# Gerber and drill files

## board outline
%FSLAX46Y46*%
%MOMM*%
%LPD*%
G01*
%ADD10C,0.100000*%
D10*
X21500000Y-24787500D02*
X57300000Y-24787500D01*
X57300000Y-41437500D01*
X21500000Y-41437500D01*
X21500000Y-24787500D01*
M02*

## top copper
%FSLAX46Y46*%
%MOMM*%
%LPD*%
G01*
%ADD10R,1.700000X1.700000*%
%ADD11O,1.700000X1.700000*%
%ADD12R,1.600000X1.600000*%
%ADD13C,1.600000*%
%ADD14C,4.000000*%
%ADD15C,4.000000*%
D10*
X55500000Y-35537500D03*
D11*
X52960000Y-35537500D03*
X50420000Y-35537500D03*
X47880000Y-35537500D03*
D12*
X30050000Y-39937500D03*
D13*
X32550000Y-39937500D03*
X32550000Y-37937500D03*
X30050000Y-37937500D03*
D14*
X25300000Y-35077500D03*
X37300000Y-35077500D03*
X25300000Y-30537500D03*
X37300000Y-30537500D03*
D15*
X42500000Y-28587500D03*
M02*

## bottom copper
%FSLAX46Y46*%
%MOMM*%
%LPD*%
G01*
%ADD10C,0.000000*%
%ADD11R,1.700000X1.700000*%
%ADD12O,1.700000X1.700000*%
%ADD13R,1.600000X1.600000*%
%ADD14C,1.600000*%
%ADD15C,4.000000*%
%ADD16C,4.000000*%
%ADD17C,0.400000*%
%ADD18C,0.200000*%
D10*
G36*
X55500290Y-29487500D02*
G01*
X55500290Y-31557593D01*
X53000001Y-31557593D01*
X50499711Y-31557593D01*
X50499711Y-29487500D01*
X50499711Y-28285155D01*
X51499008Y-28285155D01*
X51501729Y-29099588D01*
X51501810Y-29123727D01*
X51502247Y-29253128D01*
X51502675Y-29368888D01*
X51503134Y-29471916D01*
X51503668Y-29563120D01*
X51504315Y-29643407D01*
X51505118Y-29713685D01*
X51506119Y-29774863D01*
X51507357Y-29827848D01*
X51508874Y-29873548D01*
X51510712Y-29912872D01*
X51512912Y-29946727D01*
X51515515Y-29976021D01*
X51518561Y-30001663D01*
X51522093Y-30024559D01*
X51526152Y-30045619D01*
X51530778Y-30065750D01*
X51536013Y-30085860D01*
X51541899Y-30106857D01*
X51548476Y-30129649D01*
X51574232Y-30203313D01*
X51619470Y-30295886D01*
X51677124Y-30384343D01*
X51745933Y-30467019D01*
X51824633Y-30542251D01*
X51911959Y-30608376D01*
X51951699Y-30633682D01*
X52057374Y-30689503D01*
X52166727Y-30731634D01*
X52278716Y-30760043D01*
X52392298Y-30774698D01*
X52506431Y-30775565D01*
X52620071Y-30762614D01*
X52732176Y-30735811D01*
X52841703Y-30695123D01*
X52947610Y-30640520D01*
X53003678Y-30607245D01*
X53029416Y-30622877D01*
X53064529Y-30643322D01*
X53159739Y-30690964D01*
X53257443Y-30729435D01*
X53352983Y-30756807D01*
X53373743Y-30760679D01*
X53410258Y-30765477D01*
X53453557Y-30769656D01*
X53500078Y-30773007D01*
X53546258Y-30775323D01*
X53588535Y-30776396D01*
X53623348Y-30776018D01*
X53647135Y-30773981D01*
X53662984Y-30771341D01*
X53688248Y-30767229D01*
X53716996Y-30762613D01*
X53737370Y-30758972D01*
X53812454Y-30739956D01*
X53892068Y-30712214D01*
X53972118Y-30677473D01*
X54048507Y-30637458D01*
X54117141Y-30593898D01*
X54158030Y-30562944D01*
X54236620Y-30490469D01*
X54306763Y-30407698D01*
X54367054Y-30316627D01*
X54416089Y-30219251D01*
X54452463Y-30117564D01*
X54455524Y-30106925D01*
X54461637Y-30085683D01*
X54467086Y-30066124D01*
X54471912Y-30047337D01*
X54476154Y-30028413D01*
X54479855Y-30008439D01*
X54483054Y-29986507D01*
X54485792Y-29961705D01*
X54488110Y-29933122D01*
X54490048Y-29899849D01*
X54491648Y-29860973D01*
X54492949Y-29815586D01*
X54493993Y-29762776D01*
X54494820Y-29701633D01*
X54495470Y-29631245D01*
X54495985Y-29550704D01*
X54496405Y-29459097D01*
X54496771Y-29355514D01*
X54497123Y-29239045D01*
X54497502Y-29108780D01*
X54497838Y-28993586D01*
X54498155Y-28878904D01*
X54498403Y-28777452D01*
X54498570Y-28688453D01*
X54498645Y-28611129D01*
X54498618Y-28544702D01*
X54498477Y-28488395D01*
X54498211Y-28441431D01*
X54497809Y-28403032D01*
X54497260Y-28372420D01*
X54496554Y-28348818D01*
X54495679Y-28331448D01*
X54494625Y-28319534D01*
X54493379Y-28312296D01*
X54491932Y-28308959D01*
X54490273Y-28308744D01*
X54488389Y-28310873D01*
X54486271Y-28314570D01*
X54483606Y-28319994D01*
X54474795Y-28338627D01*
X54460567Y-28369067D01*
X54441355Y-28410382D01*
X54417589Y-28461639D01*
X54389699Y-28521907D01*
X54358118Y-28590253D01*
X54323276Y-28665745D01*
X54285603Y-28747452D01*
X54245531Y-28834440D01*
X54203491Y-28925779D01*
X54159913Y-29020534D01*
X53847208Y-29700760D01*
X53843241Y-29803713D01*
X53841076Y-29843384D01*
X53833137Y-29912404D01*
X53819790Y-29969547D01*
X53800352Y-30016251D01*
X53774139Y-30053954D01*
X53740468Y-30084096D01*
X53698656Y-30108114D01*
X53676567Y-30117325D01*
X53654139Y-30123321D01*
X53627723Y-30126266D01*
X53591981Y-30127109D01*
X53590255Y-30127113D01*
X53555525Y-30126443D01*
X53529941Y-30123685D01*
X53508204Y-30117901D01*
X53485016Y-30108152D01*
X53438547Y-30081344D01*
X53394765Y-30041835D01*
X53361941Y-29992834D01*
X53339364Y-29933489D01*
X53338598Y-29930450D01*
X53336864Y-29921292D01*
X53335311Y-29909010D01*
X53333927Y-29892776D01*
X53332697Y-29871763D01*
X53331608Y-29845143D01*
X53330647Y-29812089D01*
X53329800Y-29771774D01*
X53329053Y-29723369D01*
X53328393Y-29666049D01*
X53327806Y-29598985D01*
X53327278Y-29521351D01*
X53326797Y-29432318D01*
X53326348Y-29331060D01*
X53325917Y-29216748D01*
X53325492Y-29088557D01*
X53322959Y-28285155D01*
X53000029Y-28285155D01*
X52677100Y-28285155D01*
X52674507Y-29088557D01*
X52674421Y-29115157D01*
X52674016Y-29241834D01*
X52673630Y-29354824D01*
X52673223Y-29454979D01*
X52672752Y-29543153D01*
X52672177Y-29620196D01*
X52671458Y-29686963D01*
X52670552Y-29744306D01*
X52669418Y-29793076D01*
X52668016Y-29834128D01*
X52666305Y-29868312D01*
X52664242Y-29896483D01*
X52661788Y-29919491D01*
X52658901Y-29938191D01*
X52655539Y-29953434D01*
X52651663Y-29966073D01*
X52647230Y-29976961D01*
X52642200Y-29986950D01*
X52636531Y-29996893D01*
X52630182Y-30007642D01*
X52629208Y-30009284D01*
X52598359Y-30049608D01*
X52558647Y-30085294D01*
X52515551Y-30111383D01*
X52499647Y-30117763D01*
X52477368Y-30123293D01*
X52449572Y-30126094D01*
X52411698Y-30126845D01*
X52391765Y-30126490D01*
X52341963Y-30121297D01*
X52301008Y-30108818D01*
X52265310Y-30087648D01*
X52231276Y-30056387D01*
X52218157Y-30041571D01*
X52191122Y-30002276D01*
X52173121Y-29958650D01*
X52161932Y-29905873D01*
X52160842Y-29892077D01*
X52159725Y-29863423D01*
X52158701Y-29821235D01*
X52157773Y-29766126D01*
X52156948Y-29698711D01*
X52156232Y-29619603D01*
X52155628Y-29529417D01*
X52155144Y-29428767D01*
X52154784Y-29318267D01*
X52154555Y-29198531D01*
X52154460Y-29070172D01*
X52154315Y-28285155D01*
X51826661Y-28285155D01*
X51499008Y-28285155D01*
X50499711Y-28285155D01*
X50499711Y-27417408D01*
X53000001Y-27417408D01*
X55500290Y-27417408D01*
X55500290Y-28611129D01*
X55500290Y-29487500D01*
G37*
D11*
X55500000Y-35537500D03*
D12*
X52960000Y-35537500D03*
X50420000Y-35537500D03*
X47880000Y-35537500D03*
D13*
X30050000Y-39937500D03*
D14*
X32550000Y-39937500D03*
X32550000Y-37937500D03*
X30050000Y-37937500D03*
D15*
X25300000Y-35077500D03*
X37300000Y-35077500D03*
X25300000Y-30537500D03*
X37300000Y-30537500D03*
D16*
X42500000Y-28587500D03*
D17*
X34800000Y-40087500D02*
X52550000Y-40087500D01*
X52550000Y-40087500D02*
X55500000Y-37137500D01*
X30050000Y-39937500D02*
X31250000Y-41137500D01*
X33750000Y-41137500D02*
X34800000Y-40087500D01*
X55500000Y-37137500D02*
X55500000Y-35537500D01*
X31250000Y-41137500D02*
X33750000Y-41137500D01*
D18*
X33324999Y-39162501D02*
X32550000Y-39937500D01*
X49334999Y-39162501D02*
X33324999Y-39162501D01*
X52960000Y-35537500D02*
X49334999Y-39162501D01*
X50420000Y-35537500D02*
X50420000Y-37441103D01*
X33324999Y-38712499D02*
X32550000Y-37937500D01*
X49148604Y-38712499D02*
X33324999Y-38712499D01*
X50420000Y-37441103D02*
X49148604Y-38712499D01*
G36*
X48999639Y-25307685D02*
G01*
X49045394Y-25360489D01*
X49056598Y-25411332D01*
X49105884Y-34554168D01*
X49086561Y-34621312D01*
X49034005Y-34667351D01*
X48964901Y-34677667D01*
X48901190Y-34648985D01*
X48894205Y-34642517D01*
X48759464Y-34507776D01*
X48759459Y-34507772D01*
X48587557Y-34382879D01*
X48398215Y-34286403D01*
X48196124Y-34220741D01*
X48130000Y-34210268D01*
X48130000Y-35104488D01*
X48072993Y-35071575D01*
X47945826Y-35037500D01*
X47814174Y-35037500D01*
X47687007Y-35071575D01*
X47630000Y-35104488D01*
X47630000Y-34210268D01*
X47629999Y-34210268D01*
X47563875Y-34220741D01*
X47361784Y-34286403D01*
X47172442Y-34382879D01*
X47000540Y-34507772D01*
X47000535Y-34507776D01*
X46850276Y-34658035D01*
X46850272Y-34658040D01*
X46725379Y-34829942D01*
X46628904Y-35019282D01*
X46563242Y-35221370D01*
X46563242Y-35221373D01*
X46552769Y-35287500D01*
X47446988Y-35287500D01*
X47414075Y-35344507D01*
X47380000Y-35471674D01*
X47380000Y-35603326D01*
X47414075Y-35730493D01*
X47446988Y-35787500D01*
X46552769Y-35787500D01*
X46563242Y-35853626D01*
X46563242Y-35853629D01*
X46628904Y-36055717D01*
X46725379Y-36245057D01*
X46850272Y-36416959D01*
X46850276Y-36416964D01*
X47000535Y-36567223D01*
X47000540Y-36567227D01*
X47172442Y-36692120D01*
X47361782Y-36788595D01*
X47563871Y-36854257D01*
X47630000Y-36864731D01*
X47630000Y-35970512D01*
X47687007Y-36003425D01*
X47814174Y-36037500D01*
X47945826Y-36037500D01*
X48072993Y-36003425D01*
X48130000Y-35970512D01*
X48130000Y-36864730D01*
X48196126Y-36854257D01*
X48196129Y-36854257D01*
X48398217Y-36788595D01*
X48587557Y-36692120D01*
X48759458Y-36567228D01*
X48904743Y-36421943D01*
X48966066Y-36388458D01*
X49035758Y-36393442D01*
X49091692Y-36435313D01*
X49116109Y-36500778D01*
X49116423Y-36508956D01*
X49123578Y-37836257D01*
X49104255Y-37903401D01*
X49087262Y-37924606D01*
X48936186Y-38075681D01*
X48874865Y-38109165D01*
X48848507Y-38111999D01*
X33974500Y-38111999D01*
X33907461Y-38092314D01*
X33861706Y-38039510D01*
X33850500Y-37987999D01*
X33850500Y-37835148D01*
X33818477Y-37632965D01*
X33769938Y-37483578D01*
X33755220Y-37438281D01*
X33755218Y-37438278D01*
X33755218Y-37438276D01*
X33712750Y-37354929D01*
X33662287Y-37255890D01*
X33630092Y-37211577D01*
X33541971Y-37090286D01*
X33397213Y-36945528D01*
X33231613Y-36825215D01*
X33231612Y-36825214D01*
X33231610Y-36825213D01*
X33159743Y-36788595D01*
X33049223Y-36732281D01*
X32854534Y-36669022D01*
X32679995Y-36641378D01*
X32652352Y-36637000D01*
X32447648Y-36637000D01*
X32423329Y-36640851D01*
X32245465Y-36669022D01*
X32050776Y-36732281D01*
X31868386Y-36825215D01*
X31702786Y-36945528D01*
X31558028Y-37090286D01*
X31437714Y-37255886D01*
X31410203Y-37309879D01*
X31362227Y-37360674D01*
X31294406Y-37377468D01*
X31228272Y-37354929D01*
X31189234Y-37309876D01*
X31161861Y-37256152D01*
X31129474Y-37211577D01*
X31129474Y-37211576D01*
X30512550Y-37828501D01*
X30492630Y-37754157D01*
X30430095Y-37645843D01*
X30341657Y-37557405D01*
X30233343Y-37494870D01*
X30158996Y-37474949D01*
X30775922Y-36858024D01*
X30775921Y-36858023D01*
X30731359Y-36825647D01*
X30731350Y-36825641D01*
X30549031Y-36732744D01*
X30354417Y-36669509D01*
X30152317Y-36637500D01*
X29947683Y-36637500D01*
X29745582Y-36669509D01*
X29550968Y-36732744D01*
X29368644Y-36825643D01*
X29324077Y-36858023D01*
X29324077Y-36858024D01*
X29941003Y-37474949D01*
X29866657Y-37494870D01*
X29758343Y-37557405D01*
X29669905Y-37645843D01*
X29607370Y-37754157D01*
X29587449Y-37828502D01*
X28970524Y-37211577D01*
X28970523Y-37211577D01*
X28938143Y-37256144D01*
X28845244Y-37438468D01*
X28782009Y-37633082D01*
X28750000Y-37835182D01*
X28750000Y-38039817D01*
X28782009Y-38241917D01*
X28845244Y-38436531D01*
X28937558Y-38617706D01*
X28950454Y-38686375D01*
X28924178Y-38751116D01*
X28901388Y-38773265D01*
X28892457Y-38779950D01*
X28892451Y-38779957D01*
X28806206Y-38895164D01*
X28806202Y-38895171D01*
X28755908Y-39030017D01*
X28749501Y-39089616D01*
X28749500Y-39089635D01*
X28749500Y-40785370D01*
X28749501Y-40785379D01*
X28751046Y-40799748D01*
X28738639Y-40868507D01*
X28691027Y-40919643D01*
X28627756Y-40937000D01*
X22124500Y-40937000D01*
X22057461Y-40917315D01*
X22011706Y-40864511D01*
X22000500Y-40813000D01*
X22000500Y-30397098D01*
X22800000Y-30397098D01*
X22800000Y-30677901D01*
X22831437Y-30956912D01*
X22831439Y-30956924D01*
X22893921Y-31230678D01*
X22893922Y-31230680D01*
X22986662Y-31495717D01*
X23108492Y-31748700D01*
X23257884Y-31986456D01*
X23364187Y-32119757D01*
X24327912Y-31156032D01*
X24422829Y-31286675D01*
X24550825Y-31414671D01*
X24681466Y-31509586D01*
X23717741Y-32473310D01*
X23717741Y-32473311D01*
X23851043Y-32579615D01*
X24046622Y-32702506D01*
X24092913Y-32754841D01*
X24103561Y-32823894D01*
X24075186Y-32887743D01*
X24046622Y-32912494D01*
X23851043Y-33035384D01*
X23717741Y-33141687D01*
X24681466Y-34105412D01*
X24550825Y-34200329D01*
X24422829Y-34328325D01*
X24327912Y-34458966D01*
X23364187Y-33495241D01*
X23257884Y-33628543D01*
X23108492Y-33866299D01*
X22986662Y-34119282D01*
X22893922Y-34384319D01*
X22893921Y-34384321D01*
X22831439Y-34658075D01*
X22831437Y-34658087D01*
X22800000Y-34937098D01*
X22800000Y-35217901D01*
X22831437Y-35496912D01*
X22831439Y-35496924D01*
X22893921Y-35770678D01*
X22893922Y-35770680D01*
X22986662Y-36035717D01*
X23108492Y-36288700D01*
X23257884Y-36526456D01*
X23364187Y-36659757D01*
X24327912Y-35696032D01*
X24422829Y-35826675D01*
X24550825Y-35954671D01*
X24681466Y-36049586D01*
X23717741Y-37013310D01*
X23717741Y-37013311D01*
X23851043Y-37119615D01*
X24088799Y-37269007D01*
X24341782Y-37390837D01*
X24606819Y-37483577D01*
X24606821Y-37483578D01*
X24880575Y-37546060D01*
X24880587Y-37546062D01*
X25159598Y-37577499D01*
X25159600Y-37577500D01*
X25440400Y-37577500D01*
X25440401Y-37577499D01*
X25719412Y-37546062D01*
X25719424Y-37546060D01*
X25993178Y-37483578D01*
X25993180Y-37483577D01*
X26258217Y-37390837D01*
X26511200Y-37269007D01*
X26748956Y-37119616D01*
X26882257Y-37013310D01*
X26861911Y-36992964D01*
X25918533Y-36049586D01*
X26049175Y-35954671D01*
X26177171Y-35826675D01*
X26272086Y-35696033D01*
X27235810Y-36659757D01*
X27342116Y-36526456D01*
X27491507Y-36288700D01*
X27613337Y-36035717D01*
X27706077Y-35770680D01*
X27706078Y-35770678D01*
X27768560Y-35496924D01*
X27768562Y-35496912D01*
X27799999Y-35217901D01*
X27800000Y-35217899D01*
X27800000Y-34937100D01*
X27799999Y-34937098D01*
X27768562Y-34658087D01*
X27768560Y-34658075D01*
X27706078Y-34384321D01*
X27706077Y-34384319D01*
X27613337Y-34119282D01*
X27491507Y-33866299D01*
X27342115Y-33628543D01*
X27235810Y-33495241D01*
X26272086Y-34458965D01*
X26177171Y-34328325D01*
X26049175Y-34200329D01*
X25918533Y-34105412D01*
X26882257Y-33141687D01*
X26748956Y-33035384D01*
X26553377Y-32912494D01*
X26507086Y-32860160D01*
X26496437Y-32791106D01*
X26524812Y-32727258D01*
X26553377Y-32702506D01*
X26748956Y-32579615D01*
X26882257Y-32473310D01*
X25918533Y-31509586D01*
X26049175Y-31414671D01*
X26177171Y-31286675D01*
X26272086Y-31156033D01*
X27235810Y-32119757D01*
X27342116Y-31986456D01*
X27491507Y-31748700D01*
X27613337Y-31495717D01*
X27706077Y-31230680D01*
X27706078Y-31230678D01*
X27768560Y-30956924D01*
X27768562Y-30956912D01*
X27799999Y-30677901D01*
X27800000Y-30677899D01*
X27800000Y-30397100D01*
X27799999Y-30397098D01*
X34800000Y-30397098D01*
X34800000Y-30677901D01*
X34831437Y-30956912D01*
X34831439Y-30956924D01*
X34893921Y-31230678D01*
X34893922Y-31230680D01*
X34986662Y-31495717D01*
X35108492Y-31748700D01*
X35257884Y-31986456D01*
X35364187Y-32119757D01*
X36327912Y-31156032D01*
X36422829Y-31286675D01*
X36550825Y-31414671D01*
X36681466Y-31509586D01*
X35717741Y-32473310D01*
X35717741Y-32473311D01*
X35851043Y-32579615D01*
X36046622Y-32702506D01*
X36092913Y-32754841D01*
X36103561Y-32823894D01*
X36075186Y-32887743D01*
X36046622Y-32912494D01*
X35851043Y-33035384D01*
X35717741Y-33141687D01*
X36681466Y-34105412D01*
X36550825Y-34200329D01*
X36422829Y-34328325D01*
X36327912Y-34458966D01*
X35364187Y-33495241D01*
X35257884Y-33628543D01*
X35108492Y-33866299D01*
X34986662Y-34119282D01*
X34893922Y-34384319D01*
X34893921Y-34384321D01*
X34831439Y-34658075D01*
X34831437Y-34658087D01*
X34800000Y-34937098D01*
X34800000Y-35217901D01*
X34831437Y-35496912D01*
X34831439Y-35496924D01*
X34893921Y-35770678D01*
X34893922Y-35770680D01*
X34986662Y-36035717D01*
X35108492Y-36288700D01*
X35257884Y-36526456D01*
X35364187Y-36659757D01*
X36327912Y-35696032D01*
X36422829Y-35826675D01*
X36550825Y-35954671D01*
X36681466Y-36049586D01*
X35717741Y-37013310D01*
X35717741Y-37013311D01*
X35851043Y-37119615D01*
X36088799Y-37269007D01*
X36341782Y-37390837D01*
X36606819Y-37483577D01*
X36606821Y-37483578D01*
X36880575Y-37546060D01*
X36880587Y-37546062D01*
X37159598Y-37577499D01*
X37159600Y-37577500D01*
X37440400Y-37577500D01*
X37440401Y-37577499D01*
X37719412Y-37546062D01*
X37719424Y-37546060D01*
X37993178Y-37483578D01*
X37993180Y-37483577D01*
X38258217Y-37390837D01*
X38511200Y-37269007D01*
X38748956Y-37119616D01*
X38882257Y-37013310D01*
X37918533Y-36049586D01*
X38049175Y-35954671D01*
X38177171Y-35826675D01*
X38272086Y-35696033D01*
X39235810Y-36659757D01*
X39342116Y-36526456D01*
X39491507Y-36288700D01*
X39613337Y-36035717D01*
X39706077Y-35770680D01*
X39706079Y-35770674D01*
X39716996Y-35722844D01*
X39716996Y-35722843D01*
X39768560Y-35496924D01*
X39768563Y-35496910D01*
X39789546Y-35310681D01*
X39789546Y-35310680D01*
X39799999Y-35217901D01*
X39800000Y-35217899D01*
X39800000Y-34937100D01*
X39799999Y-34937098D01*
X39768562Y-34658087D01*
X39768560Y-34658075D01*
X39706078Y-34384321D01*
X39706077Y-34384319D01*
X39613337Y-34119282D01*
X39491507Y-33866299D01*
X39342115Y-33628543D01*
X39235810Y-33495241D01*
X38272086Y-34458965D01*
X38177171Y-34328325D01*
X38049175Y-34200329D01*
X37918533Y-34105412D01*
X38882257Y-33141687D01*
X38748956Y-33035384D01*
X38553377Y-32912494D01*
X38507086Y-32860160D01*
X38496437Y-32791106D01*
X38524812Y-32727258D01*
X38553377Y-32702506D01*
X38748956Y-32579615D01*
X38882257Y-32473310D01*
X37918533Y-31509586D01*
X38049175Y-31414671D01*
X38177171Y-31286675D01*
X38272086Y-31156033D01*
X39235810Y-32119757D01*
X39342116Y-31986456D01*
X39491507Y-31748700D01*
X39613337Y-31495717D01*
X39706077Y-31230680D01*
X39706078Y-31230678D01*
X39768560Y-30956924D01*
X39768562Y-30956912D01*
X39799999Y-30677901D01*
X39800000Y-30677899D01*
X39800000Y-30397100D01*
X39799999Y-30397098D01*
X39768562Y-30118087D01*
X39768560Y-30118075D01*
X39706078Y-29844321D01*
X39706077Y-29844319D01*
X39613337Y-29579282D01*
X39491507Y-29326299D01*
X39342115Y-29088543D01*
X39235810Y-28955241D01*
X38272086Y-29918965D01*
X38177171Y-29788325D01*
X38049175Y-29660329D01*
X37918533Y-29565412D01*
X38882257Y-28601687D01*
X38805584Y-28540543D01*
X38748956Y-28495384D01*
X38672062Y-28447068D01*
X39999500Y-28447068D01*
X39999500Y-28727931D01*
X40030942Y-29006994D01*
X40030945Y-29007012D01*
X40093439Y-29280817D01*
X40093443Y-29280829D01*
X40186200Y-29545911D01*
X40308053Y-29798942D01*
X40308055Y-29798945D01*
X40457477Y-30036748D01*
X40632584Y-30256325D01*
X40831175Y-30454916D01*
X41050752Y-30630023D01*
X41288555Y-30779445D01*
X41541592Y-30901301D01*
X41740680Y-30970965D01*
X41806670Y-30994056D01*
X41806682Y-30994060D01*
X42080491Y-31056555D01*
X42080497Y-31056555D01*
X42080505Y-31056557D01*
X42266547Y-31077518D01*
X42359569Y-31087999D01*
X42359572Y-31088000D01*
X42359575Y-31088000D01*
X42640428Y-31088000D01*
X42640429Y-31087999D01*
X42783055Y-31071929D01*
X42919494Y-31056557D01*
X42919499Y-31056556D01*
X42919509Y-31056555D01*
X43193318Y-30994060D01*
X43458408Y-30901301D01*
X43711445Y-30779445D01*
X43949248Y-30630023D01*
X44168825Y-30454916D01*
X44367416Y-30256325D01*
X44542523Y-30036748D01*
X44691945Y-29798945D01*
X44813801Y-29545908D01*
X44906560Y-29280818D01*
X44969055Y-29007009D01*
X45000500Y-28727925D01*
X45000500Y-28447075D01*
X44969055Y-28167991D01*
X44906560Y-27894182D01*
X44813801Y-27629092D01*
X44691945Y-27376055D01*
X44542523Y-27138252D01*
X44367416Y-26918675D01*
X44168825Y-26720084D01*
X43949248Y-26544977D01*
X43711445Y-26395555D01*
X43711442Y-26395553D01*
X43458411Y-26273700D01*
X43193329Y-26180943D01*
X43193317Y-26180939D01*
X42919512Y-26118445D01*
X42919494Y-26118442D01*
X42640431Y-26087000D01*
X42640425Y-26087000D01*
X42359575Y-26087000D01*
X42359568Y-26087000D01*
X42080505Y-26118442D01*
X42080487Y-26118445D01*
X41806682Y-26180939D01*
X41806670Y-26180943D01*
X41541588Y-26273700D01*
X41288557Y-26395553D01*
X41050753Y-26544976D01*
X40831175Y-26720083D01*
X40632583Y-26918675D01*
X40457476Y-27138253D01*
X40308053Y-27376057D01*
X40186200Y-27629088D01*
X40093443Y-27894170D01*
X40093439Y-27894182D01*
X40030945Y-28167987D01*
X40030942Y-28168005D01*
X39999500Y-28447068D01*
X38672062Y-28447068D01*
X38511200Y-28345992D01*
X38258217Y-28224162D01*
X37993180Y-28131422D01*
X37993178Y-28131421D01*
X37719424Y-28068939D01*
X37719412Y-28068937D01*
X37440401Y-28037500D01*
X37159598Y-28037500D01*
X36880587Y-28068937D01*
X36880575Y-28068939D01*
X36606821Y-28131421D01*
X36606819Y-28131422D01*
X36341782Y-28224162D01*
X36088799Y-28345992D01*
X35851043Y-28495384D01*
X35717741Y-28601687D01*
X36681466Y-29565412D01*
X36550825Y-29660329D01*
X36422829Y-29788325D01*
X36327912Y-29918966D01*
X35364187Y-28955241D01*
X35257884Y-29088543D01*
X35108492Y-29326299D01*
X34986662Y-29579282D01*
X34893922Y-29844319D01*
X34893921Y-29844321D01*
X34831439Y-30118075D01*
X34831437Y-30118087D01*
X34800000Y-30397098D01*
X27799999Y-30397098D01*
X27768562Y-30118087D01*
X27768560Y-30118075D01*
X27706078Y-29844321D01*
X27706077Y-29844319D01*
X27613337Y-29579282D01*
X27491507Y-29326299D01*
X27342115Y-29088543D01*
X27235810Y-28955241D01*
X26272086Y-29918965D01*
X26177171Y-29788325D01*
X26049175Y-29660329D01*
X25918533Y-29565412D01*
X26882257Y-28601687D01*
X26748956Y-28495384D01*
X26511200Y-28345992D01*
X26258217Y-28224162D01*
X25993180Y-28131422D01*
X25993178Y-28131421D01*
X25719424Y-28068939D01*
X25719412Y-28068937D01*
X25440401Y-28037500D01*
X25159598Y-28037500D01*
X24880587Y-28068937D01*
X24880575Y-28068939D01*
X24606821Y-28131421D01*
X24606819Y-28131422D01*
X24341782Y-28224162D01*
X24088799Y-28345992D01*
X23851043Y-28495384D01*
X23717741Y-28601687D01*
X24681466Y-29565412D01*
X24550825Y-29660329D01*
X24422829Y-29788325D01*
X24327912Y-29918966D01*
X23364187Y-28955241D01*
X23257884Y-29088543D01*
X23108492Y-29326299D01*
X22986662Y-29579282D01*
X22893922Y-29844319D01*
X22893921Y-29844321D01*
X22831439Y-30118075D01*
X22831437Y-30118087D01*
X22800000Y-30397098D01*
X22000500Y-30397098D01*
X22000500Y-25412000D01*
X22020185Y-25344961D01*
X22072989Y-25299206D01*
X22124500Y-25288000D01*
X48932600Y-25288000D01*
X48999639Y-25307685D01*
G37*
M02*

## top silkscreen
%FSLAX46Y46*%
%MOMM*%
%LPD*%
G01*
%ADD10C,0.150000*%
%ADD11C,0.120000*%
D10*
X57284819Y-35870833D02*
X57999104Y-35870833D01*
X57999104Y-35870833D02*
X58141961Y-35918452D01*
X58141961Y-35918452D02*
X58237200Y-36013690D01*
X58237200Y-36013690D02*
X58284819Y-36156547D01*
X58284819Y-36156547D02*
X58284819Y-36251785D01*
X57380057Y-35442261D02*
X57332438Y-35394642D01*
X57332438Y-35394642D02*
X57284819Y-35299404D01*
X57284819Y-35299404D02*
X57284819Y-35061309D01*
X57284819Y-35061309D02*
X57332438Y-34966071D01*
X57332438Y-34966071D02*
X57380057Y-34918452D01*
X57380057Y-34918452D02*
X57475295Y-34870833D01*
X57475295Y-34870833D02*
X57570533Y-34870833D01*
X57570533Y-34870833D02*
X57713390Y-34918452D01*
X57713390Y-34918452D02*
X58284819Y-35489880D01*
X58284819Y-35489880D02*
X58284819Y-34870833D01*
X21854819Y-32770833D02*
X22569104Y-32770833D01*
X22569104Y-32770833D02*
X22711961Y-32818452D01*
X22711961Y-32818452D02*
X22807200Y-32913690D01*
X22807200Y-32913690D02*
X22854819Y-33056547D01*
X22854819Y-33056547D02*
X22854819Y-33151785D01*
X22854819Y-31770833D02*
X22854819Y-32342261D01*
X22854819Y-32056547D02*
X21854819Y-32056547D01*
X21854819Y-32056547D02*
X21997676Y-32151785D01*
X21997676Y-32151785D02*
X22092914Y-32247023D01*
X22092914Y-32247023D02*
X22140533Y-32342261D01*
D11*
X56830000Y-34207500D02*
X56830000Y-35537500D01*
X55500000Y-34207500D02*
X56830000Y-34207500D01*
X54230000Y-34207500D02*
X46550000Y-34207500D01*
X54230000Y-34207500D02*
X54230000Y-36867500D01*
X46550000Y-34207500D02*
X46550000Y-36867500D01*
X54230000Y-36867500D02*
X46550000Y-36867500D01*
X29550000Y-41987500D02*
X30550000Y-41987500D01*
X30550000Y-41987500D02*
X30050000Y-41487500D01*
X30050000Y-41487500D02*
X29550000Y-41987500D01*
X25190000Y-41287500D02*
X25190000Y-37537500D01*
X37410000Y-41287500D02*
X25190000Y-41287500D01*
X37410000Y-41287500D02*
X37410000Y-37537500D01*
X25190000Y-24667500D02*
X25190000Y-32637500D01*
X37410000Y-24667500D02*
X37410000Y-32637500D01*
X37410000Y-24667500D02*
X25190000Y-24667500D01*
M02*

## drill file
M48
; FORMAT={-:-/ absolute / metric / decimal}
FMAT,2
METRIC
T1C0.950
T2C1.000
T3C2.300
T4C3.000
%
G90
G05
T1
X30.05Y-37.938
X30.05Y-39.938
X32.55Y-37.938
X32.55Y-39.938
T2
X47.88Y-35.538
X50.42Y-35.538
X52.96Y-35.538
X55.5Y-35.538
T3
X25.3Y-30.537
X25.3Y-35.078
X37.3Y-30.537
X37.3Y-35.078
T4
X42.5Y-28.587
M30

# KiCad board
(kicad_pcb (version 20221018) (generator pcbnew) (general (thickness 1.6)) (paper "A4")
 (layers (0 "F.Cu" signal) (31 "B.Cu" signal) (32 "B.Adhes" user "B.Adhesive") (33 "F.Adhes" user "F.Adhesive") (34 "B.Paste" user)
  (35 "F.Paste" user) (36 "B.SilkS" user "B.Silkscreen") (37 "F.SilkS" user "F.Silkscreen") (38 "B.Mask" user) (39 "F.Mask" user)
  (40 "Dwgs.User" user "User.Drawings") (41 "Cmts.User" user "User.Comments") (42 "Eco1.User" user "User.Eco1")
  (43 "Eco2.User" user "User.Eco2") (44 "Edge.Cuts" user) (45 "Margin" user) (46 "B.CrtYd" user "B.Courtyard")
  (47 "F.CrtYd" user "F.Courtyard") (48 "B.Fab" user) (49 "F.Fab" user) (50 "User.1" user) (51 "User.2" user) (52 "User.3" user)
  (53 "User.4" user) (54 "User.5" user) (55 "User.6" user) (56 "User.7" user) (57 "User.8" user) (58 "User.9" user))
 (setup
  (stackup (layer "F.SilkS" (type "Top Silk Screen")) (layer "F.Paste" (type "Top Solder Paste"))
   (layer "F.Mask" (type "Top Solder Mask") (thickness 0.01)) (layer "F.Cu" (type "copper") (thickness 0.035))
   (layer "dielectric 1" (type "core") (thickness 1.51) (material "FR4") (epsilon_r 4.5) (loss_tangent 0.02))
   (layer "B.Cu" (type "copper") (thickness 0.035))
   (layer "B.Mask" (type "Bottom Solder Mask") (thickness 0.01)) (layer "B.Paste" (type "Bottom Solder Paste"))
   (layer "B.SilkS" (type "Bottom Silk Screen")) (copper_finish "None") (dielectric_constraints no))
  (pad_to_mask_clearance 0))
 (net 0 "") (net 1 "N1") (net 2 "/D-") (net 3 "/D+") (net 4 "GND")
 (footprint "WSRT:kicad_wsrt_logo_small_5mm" (layer "F.Cu") (at 52.999711 29.5875)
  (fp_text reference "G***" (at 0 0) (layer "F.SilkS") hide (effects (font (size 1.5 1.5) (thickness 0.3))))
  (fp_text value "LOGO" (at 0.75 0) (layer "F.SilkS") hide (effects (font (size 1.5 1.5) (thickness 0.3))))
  (fp_poly
   (pts (xy -2.5 -0.1) (xy -2.5 1.970093) (xy 0.00029 1.970093) (xy 2.500579 1.970093) (xy 2.500579 -0.1) (xy 2.500579 -0.976371)
    (xy 1.498934 -0.976371) (xy 1.498859 -0.899047) (xy 1.498692 -0.810048) (xy 1.498444 -0.708596) (xy 1.498127 -0.593914)
    (xy 1.497791 -0.47872) (xy 1.497412 -0.348455) (xy 1.49706 -0.231986) (xy 1.496694 -0.128403) (xy 1.496274 -0.036796)
    (xy 1.495759 0.043745) (xy 1.495109 0.114133) (xy 1.494282 0.175276) (xy 1.493238 0.228086) (xy 1.491937 0.273473)
    (xy 1.490337 0.312349) (xy 1.488399 0.345622) (xy 1.486081 0.374205) (xy 1.483343 0.399007) (xy 1.480144 0.420939)
    (xy 1.476443 0.440913) (xy 1.472201 0.459837) (xy 1.467375 0.478624) (xy 1.461926 0.498183) (xy 1.455813 0.519425)
    (xy 1.452752 0.530064) (xy 1.416378 0.631751) (xy 1.367343 0.729127) (xy 1.307052 0.820198) (xy 1.236909 0.902969)
    (xy 1.158319 0.975444) (xy 1.11743 1.006398) (xy 1.048796 1.049958) (xy 0.972407 1.089973) (xy 0.892357 1.124714) (xy 0.812743 1.152456)
    (xy 0.737659 1.171472) (xy 0.717285 1.175113) (xy 0.688537 1.179729) (xy 0.663273 1.183841) (xy 0.647424 1.186481)
    (xy 0.623637 1.188518) (xy 0.588824 1.188896) (xy 0.546547 1.187823) (xy 0.500367 1.185507) (xy 0.453846 1.182156)
    (xy 0.410547 1.177977) (xy 0.374032 1.173179) (xy 0.353272 1.169307) (xy 0.257732 1.141935) (xy 0.160028 1.103464)
    (xy 0.064818 1.055822) (xy 0.029705 1.035377) (xy 0.003967 1.019745) (xy -0.052101 1.05302) (xy -0.158008 1.107623)
    (xy -0.267535 1.148311) (xy -0.37964 1.175114) (xy -0.49328 1.188065) (xy -0.607413 1.187198) (xy -0.720995 1.172543)
    (xy -0.832984 1.144134) (xy -0.942337 1.102003) (xy -1.048012 1.046182) (xy -1.087752 1.020876) (xy -1.175078 0.954751)
    (xy -1.253778 0.879519) (xy -1.322587 0.796843) (xy -1.380241 0.708386) (xy -1.425479 0.615813) (xy -1.451235 0.542149)
    (xy -1.457812 0.519357) (xy -1.463698 0.49836) (xy -1.468933 0.47825) (xy -1.473559 0.458119) (xy -1.477618 0.437059)
    (xy -1.48115 0.414163) (xy -1.484196 0.388521) (xy -1.486799 0.359227) (xy -1.488999 0.325372) (xy -1.490837 0.286048)
    (xy -1.492354 0.240348) (xy -1.493592 0.187363) (xy -1.494593 0.126185) (xy -1.495396 0.055907) (xy -1.496043 -0.02438)
    (xy -1.496577 -0.115584) (xy -1.497036 -0.218612) (xy -1.497464 -0.334372) (xy -1.497901 -0.463773) (xy -1.497982 -0.487912)
    (xy -1.500703 -1.302345) (xy -1.17305 -1.302345) (xy -0.845396 -1.302345) (xy -0.845251 -0.517328) (xy -0.845156 -0.388969)
    (xy -0.844927 -0.269233) (xy -0.844567 -0.158733) (xy -0.844083 -0.058083) (xy -0.843479 0.032103) (xy -0.842763 0.111211)
    (xy -0.841938 0.178626) (xy -0.84101 0.233735) (xy -0.839986 0.275923) (xy -0.838869 0.304577) (xy -0.837779 0.318373)
    (xy -0.82659 0.37115) (xy -0.808589 0.414776) (xy -0.781554 0.454071) (xy -0.768435 0.468887) (xy -0.734401 0.500148)
    (xy -0.698703 0.521318) (xy -0.657748 0.533797) (xy -0.607946 0.53899) (xy -0.588013 0.539345) (xy -0.550139 0.538594)
    (xy -0.522343 0.535793) (xy -0.500064 0.530263) (xy -0.48416 0.523883) (xy -0.441064 0.497794) (xy -0.401352 0.462108)
    (xy -0.370503 0.421784) (xy -0.369529 0.420142) (xy -0.36318 0.409393) (xy -0.357511 0.39945) (xy -0.352481 0.389461)
    (xy -0.348048 0.378573) (xy -0.344172 0.365934) (xy -0.34081 0.350691) (xy -0.337923 0.331991) (xy -0.335469 0.308983)
    (xy -0.333406 0.280812) (xy -0.331695 0.246628) (xy -0.330293 0.205576) (xy -0.329159 0.156806) (xy -0.328253 0.099463)
    (xy -0.327534 0.032696) (xy -0.326959 -0.044347) (xy -0.326488 -0.132521) (xy -0.326081 -0.232676) (xy -0.325695 -0.345666)
    (xy -0.32529 -0.472343) (xy -0.325204 -0.498943) (xy -0.322611 -1.302345) (xy 0.000318 -1.302345) (xy 0.323248 -1.302345)
    (xy 0.325781 -0.498943) (xy 0.326206 -0.370752) (xy 0.326637 -0.25644) (xy 0.327086 -0.155182) (xy 0.327567 -0.066149)
    (xy 0.328095 0.011485) (xy 0.328682 0.078549) (xy 0.329342 0.135869) (xy 0.330089 0.184274) (xy 0.330936 0.224589)
    (xy 0.331897 0.257643) (xy 0.332986 0.284263) (xy 0.334216 0.305276) (xy 0.3356 0.32151) (xy 0.337153 0.333792) (xy 0.338887 0.34295)
    (xy 0.339653 0.345989) (xy 0.36223 0.405334) (xy 0.395054 0.454335) (xy 0.438836 0.493844) (xy 0.485305 0.520652) (xy 0.508493 0.530401)
    (xy 0.53023 0.536185) (xy 0.555814 0.538943) (xy 0.590544 0.539613) (xy 0.59227 0.539609) (xy 0.628012 0.538766) (xy 0.654428 0.535821)
    (xy 0.676856 0.529825) (xy 0.698945 0.520614) (xy 0.740757 0.496596) (xy 0.774428 0.466454) (xy 0.800641 0.428751)
    (xy 0.820079 0.382047) (xy 0.833426 0.324904) (xy 0.841365 0.255884) (xy 0.84353 0.216213) (xy 0.847497 0.11326) (xy 1.160202 -0.566966)
    (xy 1.20378 -0.661721) (xy 1.24582 -0.75306) (xy 1.285892 -0.840048) (xy 1.323565 -0.921755) (xy 1.358407 -0.997247)
    (xy 1.389988 -1.065593) (xy 1.417878 -1.125861) (xy 1.441644 -1.177118) (xy 1.460856 -1.218433) (xy 1.475084 -1.248873)
    (xy 1.483895 -1.267506) (xy 1.48656 -1.27293) (xy 1.488678 -1.276627) (xy 1.490562 -1.278756) (xy 1.492221 -1.278541)
    (xy 1.493668 -1.275204) (xy 1.494914 -1.267966) (xy 1.495968 -1.256052) (xy 1.496843 -1.238682) (xy 1.497549 -1.21508)
    (xy 1.498098 -1.184468) (xy 1.4985 -1.146069) (xy 1.498766 -1.099105) (xy 1.498907 -1.042798) (xy 1.498934 -0.976371)
    (xy 2.500579 -0.976371) (xy 2.500579 -2.170092) (xy 0.00029 -2.170092) (xy -2.5 -2.170092))
   (stroke (width 0) (type solid)) (fill solid) (layer "B.Cu")))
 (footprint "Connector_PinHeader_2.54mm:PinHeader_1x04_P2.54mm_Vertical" (layer "F.Cu") (at 55.5 35.5375 -90)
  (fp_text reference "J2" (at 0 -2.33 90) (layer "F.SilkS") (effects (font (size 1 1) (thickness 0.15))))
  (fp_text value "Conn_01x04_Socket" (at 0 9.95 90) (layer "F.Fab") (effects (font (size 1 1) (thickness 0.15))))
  (fp_line (start -1.33 -1.33) (end 0 -1.33) (stroke (width 0.12) (type solid)) (layer "F.SilkS"))
  (fp_line (start -1.33 0) (end -1.33 -1.33) (stroke (width 0.12) (type solid)) (layer "F.SilkS"))
  (fp_line (start -1.33 1.27) (end -1.33 8.95) (stroke (width 0.12) (type solid)) (layer "F.SilkS"))
  (fp_line (start -1.33 1.27) (end 1.33 1.27) (stroke (width 0.12) (type solid)) (layer "F.SilkS"))
  (fp_line (start -1.33 8.95) (end 1.33 8.95) (stroke (width 0.12) (type solid)) (layer "F.SilkS"))
  (fp_line (start 1.33 1.27) (end 1.33 8.95) (stroke (width 0.12) (type solid)) (layer "F.SilkS"))
  (pad "1" thru_hole rect (at 0 0 270) (size 1.7 1.7) (drill 1) (layers "*.Cu" "*.Mask") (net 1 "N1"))
  (pad "2" thru_hole oval (at 0 2.54 270) (size 1.7 1.7) (drill 1) (layers "*.Cu" "*.Mask") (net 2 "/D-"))
  (pad "3" thru_hole oval (at 0 5.08 270) (size 1.7 1.7) (drill 1) (layers "*.Cu" "*.Mask") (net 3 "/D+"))
  (pad "4" thru_hole oval (at 0 7.62 270) (size 1.7 1.7) (drill 1) (layers "*.Cu" "*.Mask") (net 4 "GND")))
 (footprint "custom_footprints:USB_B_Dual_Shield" (layer "F.Cu") (at 30.05 39.9375 90)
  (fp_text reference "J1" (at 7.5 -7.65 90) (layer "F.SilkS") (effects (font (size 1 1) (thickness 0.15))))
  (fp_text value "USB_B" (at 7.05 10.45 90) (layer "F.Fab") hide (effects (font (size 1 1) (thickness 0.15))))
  (fp_line (start -2.05 -0.5) (end -2.05 0.5) (stroke (width 0.12) (type solid)) (layer "F.SilkS"))
  (fp_line (start -2.05 0.5) (end -1.55 0) (stroke (width 0.12) (type solid)) (layer "F.SilkS"))
  (fp_line (start -1.55 0) (end -2.05 -0.5) (stroke (width 0.12) (type solid)) (layer "F.SilkS"))
  (fp_line (start -1.35 -4.86) (end 2.4 -4.86) (stroke (width 0.12) (type solid)) (layer "F.SilkS"))
  (fp_line (start -1.35 7.36) (end -1.35 -4.86) (stroke (width 0.12) (type solid)) (layer "F.SilkS"))
  (fp_line (start -1.35 7.36) (end 2.4 7.36) (stroke (width 0.12) (type solid)) (layer "F.SilkS"))
  (fp_line (start 15.27 -4.86) (end 7.3 -4.86) (stroke (width 0.12) (type solid)) (layer "F.SilkS"))
  (fp_line (start 15.27 7.36) (end 7.3 7.36) (stroke (width 0.12) (type solid)) (layer "F.SilkS"))
  (fp_line (start 15.27 7.36) (end 15.27 -4.86) (stroke (width 0.12) (type solid)) (layer "F.SilkS"))
  (pad "1" thru_hole rect (at 0 0 180) (size 1.6 1.6) (drill 0.95) (layers "*.Cu" "*.Mask") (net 1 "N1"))
  (pad "2" thru_hole circle (at 0 2.5 180) (size 1.6 1.6) (drill 0.95) (layers "*.Cu" "*.Mask") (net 2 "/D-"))
  (pad "3" thru_hole circle (at 2 2.5 180) (size 1.6 1.6) (drill 0.95) (layers "*.Cu" "*.Mask") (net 3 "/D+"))
  (pad "4" thru_hole circle (at 2 0 180) (size 1.6 1.6) (drill 0.95) (layers "*.Cu" "*.Mask") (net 4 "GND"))
  (pad "5" thru_hole circle (at 4.86 -4.75 180) (size 4 4) (drill 2.3) (layers "*.Cu" "*.Mask") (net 4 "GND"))
  (pad "5" thru_hole circle (at 4.86 7.25 180) (size 4 4) (drill 2.3) (layers "*.Cu" "*.Mask") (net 4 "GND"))
  (pad "5" thru_hole circle (at 9.4 -4.75 180) (size 4 4) (drill 2.3) (layers "*.Cu" "*.Mask") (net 4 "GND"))
  (pad "5" thru_hole circle (at 9.4 7.25 180) (size 4 4) (drill 2.3) (layers "*.Cu" "*.Mask") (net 4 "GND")))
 (gr_rect (start 21.5 24.7875) (end 57.3 41.4375) (stroke (width 0.1) (type default)) (fill none) (layer "Edge.Cuts"))
 (via (at 42.5 28.5875) (size 4) (drill 3) (layers "F.Cu" "B.Cu") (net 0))
 (segment (start 34.8 40.0875) (end 52.55 40.0875) (width 0.4) (layer "B.Cu") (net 1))
 (segment (start 52.55 40.0875) (end 55.5 37.1375) (width 0.4) (layer "B.Cu") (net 1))
 (segment (start 30.05 39.9375) (end 31.25 41.1375) (width 0.4) (layer "B.Cu") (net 1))
 (segment (start 33.75 41.1375) (end 34.8 40.0875) (width 0.4) (layer "B.Cu") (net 1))
 (segment (start 55.5 37.1375) (end 55.5 35.5375) (width 0.4) (layer "B.Cu") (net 1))
 (segment (start 31.25 41.1375) (end 33.75 41.1375) (width 0.4) (layer "B.Cu") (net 1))
 (segment (start 33.324999 39.162501) (end 32.55 39.9375) (width 0.2) (layer "B.Cu") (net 2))
 (segment (start 49.334999 39.162501) (end 33.324999 39.162501) (width 0.2) (layer "B.Cu") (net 2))
 (segment (start 52.96 35.5375) (end 49.334999 39.162501) (width 0.2) (layer "B.Cu") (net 2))
 (segment (start 50.42 35.5375) (end 50.42 37.441103) (width 0.2) (layer "B.Cu") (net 3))
 (segment (start 33.324999 38.712499) (end 32.55 37.9375) (width 0.2) (layer "B.Cu") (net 3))
 (segment (start 49.148604 38.712499) (end 33.324999 38.712499) (width 0.2) (layer "B.Cu") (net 3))
 (segment (start 50.42 37.441103) (end 49.148604 38.712499) (width 0.2) (layer "B.Cu") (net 3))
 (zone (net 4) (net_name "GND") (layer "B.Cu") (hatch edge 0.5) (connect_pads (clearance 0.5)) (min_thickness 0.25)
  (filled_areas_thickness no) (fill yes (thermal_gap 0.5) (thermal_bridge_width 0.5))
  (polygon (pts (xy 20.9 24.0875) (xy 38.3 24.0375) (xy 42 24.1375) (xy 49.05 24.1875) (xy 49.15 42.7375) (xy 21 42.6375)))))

